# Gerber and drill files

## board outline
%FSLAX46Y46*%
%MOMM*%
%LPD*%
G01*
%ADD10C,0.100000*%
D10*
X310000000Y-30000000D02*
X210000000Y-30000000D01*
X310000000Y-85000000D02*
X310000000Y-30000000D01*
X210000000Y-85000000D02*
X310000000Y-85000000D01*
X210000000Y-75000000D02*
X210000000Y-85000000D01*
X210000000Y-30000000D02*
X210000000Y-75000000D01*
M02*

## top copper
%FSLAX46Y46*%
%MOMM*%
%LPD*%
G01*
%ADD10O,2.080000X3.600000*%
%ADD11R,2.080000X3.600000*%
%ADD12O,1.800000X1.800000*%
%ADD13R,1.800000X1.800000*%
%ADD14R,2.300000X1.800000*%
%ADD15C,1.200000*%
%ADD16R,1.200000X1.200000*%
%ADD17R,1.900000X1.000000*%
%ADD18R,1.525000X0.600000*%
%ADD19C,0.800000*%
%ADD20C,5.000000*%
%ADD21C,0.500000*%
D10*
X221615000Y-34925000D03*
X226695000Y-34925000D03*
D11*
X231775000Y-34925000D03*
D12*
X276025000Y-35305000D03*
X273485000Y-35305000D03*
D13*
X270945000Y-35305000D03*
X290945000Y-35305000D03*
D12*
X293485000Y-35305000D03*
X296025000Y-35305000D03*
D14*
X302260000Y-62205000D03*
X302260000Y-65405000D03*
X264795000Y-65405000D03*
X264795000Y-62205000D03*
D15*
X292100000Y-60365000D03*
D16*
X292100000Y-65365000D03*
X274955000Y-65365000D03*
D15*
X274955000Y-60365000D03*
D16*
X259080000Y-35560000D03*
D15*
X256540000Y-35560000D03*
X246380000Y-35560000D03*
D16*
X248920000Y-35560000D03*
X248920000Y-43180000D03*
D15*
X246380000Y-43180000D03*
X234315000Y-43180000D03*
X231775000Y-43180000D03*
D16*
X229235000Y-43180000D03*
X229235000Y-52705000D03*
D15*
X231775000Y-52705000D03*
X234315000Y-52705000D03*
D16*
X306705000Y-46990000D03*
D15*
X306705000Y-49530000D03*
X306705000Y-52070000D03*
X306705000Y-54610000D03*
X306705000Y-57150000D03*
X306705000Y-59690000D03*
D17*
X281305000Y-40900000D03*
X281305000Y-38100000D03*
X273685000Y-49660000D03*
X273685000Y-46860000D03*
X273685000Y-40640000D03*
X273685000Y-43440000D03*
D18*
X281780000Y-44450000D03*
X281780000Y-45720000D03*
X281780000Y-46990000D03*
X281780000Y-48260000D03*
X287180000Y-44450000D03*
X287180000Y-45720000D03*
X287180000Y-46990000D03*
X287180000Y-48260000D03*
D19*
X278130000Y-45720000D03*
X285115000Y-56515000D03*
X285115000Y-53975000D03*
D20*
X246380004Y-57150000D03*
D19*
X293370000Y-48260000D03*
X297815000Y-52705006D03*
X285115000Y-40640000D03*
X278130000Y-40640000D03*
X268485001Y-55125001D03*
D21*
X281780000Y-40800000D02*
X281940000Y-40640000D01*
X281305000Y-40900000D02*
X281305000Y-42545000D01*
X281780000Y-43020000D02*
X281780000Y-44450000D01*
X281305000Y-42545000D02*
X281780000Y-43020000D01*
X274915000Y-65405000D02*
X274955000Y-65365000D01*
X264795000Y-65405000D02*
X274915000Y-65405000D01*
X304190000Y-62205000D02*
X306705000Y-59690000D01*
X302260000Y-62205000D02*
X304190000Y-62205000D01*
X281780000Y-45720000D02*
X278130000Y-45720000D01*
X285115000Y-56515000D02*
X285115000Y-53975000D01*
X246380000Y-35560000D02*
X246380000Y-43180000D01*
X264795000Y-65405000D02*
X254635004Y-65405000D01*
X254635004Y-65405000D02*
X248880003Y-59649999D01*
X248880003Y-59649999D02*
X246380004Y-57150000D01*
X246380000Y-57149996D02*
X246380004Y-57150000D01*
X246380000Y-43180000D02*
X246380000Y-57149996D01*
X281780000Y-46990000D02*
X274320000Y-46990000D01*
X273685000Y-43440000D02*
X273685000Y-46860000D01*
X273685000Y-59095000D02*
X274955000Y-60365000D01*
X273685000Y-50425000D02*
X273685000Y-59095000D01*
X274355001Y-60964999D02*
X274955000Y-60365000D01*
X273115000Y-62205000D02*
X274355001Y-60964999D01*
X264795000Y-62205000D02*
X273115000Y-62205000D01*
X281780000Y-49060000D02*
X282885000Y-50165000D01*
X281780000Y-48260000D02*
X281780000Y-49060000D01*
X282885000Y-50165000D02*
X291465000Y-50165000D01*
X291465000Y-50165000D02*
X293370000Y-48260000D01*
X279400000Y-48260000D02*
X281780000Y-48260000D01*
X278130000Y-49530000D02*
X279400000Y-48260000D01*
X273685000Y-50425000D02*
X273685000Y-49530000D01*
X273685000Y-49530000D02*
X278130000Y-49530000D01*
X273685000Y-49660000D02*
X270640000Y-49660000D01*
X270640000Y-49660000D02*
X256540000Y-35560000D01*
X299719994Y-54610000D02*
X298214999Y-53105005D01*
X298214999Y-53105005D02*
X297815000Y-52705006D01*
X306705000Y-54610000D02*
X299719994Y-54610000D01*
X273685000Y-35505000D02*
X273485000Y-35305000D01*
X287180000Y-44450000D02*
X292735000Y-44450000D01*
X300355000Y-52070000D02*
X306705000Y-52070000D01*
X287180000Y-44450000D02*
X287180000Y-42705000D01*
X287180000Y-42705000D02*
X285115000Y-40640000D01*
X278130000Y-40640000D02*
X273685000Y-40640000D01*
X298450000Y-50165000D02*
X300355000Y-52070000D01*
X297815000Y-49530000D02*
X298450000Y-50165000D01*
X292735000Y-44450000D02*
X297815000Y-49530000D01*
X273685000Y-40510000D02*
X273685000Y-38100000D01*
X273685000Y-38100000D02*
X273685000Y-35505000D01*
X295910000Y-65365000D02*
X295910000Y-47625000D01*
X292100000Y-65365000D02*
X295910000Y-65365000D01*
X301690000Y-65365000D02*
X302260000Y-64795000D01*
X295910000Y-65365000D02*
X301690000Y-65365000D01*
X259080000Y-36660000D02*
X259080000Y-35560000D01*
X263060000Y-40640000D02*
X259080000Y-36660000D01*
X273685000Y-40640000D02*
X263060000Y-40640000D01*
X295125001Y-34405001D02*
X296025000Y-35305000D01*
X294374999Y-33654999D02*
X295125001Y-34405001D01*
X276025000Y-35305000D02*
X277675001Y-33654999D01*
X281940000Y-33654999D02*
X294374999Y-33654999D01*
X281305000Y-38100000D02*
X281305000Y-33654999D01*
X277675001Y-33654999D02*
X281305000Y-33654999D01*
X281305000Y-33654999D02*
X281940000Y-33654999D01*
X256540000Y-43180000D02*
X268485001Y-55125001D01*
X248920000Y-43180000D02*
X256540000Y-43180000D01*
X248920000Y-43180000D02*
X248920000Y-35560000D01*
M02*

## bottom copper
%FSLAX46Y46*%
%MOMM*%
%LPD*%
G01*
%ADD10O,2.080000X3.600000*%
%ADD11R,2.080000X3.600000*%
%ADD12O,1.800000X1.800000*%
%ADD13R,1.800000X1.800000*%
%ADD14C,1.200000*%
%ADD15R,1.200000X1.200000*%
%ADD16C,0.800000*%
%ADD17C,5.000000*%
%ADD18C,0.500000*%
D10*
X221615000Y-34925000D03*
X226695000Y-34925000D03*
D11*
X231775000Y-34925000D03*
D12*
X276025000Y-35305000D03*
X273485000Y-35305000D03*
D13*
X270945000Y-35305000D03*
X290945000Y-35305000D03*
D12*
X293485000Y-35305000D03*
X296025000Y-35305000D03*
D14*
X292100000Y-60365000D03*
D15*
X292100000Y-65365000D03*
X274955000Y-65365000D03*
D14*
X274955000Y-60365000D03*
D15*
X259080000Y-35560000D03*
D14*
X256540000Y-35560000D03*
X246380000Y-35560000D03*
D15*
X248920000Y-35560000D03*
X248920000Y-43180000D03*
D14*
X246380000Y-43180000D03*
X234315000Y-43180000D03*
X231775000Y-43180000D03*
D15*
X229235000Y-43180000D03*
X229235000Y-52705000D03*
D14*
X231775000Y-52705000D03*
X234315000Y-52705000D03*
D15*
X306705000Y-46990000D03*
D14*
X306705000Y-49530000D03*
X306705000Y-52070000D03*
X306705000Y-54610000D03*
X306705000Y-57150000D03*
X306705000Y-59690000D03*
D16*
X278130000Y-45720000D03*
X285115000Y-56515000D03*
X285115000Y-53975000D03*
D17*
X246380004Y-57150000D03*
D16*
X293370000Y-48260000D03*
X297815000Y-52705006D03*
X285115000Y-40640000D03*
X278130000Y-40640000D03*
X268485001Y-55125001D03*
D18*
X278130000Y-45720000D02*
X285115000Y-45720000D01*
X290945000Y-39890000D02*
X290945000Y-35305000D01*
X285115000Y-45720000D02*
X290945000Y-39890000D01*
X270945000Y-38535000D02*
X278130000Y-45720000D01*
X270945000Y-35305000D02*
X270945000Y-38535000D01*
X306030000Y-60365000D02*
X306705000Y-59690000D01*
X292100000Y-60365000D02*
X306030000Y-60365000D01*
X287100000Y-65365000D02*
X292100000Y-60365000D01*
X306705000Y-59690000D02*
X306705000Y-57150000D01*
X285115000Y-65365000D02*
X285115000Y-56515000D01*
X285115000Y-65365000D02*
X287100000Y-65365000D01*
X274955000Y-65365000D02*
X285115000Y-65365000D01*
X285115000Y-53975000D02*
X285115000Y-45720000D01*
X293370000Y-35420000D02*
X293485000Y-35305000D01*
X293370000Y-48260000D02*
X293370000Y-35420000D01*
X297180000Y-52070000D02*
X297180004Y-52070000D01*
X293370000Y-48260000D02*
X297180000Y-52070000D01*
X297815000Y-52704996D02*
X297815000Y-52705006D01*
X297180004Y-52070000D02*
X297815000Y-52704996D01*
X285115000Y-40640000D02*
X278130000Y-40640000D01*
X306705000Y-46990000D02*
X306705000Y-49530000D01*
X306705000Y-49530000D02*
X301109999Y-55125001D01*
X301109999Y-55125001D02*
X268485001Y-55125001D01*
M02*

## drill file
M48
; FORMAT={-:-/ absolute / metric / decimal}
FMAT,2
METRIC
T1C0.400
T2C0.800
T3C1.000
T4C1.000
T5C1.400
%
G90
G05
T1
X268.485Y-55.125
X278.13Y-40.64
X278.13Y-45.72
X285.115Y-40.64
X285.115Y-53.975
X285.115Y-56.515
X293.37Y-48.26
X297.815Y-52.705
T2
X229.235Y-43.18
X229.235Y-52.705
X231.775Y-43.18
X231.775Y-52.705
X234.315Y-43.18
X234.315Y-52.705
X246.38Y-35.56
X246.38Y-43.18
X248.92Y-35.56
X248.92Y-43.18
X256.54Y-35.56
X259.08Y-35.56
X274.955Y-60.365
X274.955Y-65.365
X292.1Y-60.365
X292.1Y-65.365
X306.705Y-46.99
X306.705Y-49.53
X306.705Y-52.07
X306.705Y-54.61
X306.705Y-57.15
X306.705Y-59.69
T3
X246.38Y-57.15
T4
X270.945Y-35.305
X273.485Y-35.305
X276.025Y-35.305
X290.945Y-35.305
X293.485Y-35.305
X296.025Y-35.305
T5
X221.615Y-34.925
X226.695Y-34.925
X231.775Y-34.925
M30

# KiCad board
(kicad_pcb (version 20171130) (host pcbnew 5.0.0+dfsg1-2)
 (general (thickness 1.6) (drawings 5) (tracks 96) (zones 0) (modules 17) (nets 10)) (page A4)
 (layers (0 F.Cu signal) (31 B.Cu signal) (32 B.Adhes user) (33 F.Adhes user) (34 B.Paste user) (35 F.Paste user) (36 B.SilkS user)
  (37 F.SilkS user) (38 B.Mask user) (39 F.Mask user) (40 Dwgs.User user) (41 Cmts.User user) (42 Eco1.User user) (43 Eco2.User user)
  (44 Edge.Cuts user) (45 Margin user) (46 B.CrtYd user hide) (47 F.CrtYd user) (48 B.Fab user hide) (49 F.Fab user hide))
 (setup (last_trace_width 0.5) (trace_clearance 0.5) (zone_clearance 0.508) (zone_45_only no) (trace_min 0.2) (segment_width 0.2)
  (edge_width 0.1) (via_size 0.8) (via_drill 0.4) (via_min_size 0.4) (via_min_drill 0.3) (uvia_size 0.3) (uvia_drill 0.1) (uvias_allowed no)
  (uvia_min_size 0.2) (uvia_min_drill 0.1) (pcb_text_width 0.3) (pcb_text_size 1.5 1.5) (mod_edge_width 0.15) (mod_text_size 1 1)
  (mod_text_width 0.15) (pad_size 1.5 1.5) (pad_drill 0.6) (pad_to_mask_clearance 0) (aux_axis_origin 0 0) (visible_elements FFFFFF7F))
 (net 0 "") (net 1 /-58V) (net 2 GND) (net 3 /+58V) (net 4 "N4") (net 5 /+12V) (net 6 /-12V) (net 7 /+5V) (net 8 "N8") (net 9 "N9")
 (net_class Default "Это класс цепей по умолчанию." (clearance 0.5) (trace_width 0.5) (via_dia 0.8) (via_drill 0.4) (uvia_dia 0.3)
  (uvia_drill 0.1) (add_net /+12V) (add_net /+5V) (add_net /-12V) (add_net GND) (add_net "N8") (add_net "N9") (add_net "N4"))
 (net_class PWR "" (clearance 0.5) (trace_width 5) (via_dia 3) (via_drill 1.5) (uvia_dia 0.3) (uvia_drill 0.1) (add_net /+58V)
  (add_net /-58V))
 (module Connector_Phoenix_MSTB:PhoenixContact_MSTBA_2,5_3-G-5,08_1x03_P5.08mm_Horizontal (layer F.Cu) (at 231.775 34.925 180)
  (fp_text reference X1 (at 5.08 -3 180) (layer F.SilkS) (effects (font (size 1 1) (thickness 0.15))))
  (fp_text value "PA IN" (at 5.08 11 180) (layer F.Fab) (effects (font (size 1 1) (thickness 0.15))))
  (pad 3 thru_hole oval (at 10.16 0 180) (size 2.08 3.6) (drill 1.4) (layers *.Cu *.Mask) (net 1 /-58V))
  (pad 2 thru_hole oval (at 5.08 0 180) (size 2.08 3.6) (drill 1.4) (layers *.Cu *.Mask) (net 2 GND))
  (pad 1 thru_hole rect (at 0 0 180) (size 2.08 3.6) (drill 1.4) (layers *.Cu *.Mask) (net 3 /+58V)))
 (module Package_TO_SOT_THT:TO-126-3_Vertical (layer F.Cu) (at 270.945 35.305)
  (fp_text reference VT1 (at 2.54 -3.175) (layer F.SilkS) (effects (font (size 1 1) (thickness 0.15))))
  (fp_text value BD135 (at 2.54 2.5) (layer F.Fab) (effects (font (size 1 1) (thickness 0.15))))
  (pad 3 thru_hole oval (at 5.08 0) (size 1.8 1.8) (drill 1) (layers *.Cu *.Mask) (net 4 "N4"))
  (pad 2 thru_hole oval (at 2.54 0) (size 1.8 1.8) (drill 1) (layers *.Cu *.Mask) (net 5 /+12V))
  (pad 1 thru_hole rect (at 0 0) (size 1.8 1.8) (drill 1) (layers *.Cu *.Mask) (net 2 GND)))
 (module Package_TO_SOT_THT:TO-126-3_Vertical (layer F.Cu) (at 290.945 35.305)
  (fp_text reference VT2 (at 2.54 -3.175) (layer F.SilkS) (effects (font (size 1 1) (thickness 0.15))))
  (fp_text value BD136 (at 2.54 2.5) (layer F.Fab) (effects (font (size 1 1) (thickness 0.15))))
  (pad 1 thru_hole rect (at 0 0) (size 1.8 1.8) (drill 1) (layers *.Cu *.Mask) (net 2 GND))
  (pad 2 thru_hole oval (at 2.54 0) (size 1.8 1.8) (drill 1) (layers *.Cu *.Mask) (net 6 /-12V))
  (pad 3 thru_hole oval (at 5.08 0) (size 1.8 1.8) (drill 1) (layers *.Cu *.Mask) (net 4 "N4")))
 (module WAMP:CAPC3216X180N (layer F.Cu) (at 302.26 63.805 180)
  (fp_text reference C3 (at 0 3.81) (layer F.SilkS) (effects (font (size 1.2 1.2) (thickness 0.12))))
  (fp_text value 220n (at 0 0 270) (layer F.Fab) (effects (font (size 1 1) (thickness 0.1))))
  (pad 2 smd rect (at 0 1.6 180) (size 2.3 1.8) (layers F.Cu F.Paste F.Mask) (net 2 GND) (solder_mask_margin 0.2))
  (pad 1 smd rect (at 0 -1.6 180) (size 2.3 1.8) (layers F.Cu F.Paste F.Mask) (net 5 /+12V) (solder_mask_margin 0.2)))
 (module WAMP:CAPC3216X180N (layer F.Cu) (at 264.795 63.805 180)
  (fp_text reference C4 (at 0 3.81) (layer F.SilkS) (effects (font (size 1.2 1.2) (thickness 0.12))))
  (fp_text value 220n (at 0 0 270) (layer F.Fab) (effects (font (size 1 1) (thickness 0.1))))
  (pad 1 smd rect (at 0 -1.6 180) (size 2.3 1.8) (layers F.Cu F.Paste F.Mask) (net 2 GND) (solder_mask_margin 0.2))
  (pad 2 smd rect (at 0 1.6 180) (size 2.3 1.8) (layers F.Cu F.Paste F.Mask) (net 6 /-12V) (solder_mask_margin 0.2)))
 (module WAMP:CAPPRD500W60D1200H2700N (layer F.Cu) (at 292.1 62.865 180)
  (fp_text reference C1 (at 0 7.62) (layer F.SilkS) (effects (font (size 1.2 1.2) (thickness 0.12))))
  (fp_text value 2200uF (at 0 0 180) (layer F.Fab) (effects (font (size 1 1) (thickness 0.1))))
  (pad 2 thru_hole circle (at 0 2.5 180) (size 1.2 1.2) (drill 0.8) (layers F&B.Cu *.Paste *.Mask) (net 2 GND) (solder_mask_margin 0.2))
  (pad 1 thru_hole rect (at 0 -2.5 180) (size 1.2 1.2) (drill 0.8) (layers F&B.Cu *.Paste *.Mask) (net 5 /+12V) (solder_mask_margin 0.2)))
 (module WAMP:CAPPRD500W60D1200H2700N (layer F.Cu) (at 274.955 62.865 180)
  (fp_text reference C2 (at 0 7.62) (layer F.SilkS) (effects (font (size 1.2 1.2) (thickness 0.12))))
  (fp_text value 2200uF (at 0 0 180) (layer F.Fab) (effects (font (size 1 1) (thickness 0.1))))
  (pad 1 thru_hole rect (at 0 -2.5 180) (size 1.2 1.2) (drill 0.8) (layers F&B.Cu *.Paste *.Mask) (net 2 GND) (solder_mask_margin 0.2))
  (pad 2 thru_hole circle (at 0 2.5 180) (size 1.2 1.2) (drill 0.8) (layers F&B.Cu *.Paste *.Mask) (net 6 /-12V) (solder_mask_margin 0.2)))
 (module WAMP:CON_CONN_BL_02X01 (layer F.Cu) (at 257.81 35.56 270)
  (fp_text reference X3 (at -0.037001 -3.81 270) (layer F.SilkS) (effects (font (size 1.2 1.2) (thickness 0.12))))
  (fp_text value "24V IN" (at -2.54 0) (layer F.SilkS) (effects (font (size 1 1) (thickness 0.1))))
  (pad 1 thru_hole rect (at 0 -1.27 270) (size 1.2 1.2) (drill 0.8) (layers F&B.Cu *.Paste *.Mask) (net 5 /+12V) (solder_mask_margin 0.2))
  (pad 2 thru_hole circle (at 0 1.27 270) (size 1.2 1.2) (drill 0.8) (layers F&B.Cu *.Paste *.Mask) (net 6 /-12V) (solder_mask_margin 0.2)))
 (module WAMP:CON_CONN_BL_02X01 (layer F.Cu) (at 247.65 35.56 270)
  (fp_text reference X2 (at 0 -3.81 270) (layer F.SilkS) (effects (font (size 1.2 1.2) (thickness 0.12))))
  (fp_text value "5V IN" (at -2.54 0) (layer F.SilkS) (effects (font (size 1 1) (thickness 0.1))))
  (pad 2 thru_hole circle (at 0 1.27 270) (size 1.2 1.2) (drill 0.8) (layers F&B.Cu *.Paste *.Mask) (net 2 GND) (solder_mask_margin 0.2))
  (pad 1 thru_hole rect (at 0 -1.27 270) (size 1.2 1.2) (drill 0.8) (layers F&B.Cu *.Paste *.Mask) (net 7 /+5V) (solder_mask_margin 0.2)))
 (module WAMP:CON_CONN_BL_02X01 (layer F.Cu) (at 247.65 43.18 270)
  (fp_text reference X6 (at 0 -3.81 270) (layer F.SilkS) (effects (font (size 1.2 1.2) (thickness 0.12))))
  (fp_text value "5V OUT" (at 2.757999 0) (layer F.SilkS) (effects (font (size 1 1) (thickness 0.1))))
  (pad 1 thru_hole rect (at 0 -1.27 270) (size 1.2 1.2) (drill 0.8) (layers F&B.Cu *.Paste *.Mask) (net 7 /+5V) (solder_mask_margin 0.2))
  (pad 2 thru_hole circle (at 0 1.27 270) (size 1.2 1.2) (drill 0.8) (layers F&B.Cu *.Paste *.Mask) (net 2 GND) (solder_mask_margin 0.2)))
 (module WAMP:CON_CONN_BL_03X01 (layer F.Cu) (at 231.775 43.18 90)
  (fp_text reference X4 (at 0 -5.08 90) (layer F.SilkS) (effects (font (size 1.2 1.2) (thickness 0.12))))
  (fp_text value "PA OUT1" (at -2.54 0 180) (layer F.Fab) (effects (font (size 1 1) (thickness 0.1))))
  (pad 3 thru_hole circle (at 0 2.54 90) (size 1.2 1.2) (drill 0.8) (layers F&B.Cu *.Paste *.Mask) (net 1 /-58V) (solder_mask_margin 0.2))
  (pad 2 thru_hole circle (at 0 0 90) (size 1.2 1.2) (drill 0.8) (layers F&B.Cu *.Paste *.Mask) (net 2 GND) (solder_mask_margin 0.2))
  (pad 1 thru_hole rect (at 0 -2.54 90) (size 1.2 1.2) (drill 0.8) (layers F&B.Cu *.Paste *.Mask) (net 3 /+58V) (solder_mask_margin 0.2)))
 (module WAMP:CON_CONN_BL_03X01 (layer F.Cu) (at 231.775 52.705 90)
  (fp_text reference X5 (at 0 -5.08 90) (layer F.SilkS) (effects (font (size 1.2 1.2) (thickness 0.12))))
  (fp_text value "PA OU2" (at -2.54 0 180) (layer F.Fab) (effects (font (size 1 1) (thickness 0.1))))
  (pad 1 thru_hole rect (at 0 -2.54 90) (size 1.2 1.2) (drill 0.8) (layers F&B.Cu *.Paste *.Mask) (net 3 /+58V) (solder_mask_margin 0.2))
  (pad 2 thru_hole circle (at 0 0 90) (size 1.2 1.2) (drill 0.8) (layers F&B.Cu *.Paste *.Mask) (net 2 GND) (solder_mask_margin 0.2))
  (pad 3 thru_hole circle (at 0 2.54 90) (size 1.2 1.2) (drill 0.8) (layers F&B.Cu *.Paste *.Mask) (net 1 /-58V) (solder_mask_margin 0.2)))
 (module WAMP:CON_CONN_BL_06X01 (layer F.Cu) (at 306.705 53.34)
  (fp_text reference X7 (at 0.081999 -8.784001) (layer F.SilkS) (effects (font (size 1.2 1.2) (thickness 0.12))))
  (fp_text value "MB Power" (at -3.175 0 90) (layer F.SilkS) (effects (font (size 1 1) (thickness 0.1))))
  (pad 1 thru_hole rect (at 0 -6.35) (size 1.2 1.2) (drill 0.8) (layers F&B.Cu *.Paste *.Mask) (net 7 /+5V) (solder_mask_margin 0.2))
  (pad 2 thru_hole circle (at 0 -3.81) (size 1.2 1.2) (drill 0.8) (layers F&B.Cu *.Paste *.Mask) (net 7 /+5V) (solder_mask_margin 0.2))
  (pad 3 thru_hole circle (at 0 -1.27) (size 1.2 1.2) (drill 0.8) (layers F&B.Cu *.Paste *.Mask) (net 5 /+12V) (solder_mask_margin 0.2))
  (pad 4 thru_hole circle (at 0 1.27) (size 1.2 1.2) (drill 0.8) (layers F&B.Cu *.Paste *.Mask) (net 6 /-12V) (solder_mask_margin 0.2))
  (pad 5 thru_hole circle (at 0 3.81) (size 1.2 1.2) (drill 0.8) (layers F&B.Cu *.Paste *.Mask) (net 2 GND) (solder_mask_margin 0.2))
  (pad 6 thru_hole circle (at 0 6.35) (size 1.2 1.2) (drill 0.8) (layers F&B.Cu *.Paste *.Mask) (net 2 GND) (solder_mask_margin 0.2)))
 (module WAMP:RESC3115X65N (layer F.Cu) (at 281.305 39.5 180)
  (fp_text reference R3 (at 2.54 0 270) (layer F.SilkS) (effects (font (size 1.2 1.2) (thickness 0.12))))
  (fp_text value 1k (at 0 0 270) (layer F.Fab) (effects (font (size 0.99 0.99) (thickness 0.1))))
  (pad 1 smd rect (at 0 -1.4 180) (size 1.9 1) (layers F.Cu F.Paste F.Mask) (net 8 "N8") (solder_mask_margin 0.2))
  (pad 2 smd rect (at 0 1.4 180) (size 1.9 1) (layers F.Cu F.Paste F.Mask) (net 4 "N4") (solder_mask_margin 0.2)))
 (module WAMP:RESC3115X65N (layer F.Cu) (at 273.685 48.26)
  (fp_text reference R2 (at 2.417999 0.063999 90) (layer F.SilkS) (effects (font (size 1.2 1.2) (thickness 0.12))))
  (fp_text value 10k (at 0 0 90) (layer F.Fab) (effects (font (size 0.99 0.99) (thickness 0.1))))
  (pad 2 smd rect (at 0 1.4) (size 1.9 1) (layers F.Cu F.Paste F.Mask) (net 6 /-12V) (solder_mask_margin 0.2))
  (pad 1 smd rect (at 0 -1.4) (size 1.9 1) (layers F.Cu F.Paste F.Mask) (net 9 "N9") (solder_mask_margin 0.2)))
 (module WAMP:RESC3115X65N (layer F.Cu) (at 273.685 42.04)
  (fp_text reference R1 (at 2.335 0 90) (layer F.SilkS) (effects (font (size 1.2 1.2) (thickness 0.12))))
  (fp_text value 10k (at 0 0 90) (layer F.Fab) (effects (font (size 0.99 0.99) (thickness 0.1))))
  (pad 1 smd rect (at 0 -1.4) (size 1.9 1) (layers F.Cu F.Paste F.Mask) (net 5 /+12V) (solder_mask_margin 0.2))
  (pad 2 smd rect (at 0 1.4) (size 1.9 1) (layers F.Cu F.Paste F.Mask) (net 9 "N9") (solder_mask_margin 0.2)))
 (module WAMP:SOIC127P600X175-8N (layer F.Cu) (at 284.48 46.355)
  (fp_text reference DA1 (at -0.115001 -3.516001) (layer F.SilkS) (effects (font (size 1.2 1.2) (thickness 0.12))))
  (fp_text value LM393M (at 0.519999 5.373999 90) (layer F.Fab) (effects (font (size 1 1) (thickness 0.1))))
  (pad 1 smd rect (at -2.7 -1.905) (size 1.525 0.6) (layers F.Cu F.Paste F.Mask) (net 8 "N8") (solder_mask_margin 0.2))
  (pad 2 smd rect (at -2.7 -0.635) (size 1.525 0.6) (layers F.Cu F.Paste F.Mask) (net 2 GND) (solder_mask_margin 0.2))
  (pad 3 smd rect (at -2.7 0.635) (size 1.525 0.6) (layers F.Cu F.Paste F.Mask) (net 9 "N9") (solder_mask_margin 0.2))
  (pad 4 smd rect (at -2.7 1.905) (size 1.525 0.6) (layers F.Cu F.Paste F.Mask) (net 6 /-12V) (solder_mask_margin 0.2))
  (pad 8 smd rect (at 2.7 -1.905) (size 1.525 0.6) (layers F.Cu F.Paste F.Mask) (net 5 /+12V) (solder_mask_margin 0.2))
  (pad 7 smd rect (at 2.7 -0.635) (size 1.525 0.6) (layers F.Cu F.Paste F.Mask) (solder_mask_margin 0.2))
  (pad 6 smd rect (at 2.7 0.635) (size 1.525 0.6) (layers F.Cu F.Paste F.Mask) (solder_mask_margin 0.2))
  (pad 5 smd rect (at 2.7 1.905) (size 1.525 0.6) (layers F.Cu F.Paste F.Mask) (solder_mask_margin 0.2)))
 (gr_line (start 310 30) (end 210 30) (layer Edge.Cuts) (width 0.1))
 (gr_line (start 310 85) (end 310 30) (layer Edge.Cuts) (width 0.1))
 (gr_line (start 210 85) (end 310 85) (layer Edge.Cuts) (width 0.1))
 (gr_line (start 210 75) (end 210 85) (layer Edge.Cuts) (width 0.1))
 (gr_line (start 210 30) (end 210 75) (layer Edge.Cuts) (width 0.1))
 (segment (start 281.78 40.8) (end 281.94 40.64) (width 0.5) (layer F.Cu) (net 8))
 (segment (start 281.305 40.9) (end 281.305 42.545) (width 0.5) (layer F.Cu) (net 8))
 (segment (start 281.78 43.02) (end 281.78 44.45) (width 0.5) (layer F.Cu) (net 8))
 (segment (start 281.305 42.545) (end 281.78 43.02) (width 0.5) (layer F.Cu) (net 8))
 (segment (start 274.915 65.405) (end 274.955 65.365) (width 0.5) (layer F.Cu) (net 2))
 (segment (start 264.795 65.405) (end 274.915 65.405) (width 0.5) (layer F.Cu) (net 2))
 (segment (start 304.19 62.205) (end 306.705 59.69) (width 0.5) (layer F.Cu) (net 2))
 (segment (start 302.26 62.205) (end 304.19 62.205) (width 0.5) (layer F.Cu) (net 2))
 (via (at 278.13 45.72) (size 0.8) (drill 0.4) (layers F.Cu B.Cu) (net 2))
 (segment (start 281.78 45.72) (end 278.13 45.72) (width 0.5) (layer F.Cu) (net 2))
 (segment (start 278.13 45.72) (end 285.115 45.72) (width 0.5) (layer B.Cu) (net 2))
 (segment (start 290.945 39.89) (end 290.945 35.305) (width 0.5) (layer B.Cu) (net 2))
 (segment (start 285.115 45.72) (end 290.945 39.89) (width 0.5) (layer B.Cu) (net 2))
 (segment (start 270.945 38.535) (end 278.13 45.72) (width 0.5) (layer B.Cu) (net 2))
 (segment (start 270.945 35.305) (end 270.945 38.535) (width 0.5) (layer B.Cu) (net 2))
 (segment (start 306.03 60.365) (end 306.705 59.69) (width 0.5) (layer B.Cu) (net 2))
 (segment (start 292.1 60.365) (end 306.03 60.365) (width 0.5) (layer B.Cu) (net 2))
 (segment (start 287.1 65.365) (end 292.1 60.365) (width 0.5) (layer B.Cu) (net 2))
 (segment (start 306.705 59.69) (end 306.705 57.15) (width 0.5) (layer B.Cu) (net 2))
 (segment (start 285.115 65.365) (end 285.115 56.515) (width 0.5) (layer B.Cu) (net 2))
 (segment (start 285.115 65.365) (end 287.1 65.365) (width 0.5) (layer B.Cu) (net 2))
 (via (at 285.115 56.515) (size 0.8) (drill 0.4) (layers F.Cu B.Cu) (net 2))
 (segment (start 274.955 65.365) (end 285.115 65.365) (width 0.5) (layer B.Cu) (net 2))
 (via (at 285.115 53.975) (size 0.8) (drill 0.4) (layers F.Cu B.Cu) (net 2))
 (segment (start 285.115 56.515) (end 285.115 53.975) (width 0.5) (layer F.Cu) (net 2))
 (segment (start 285.115 53.975) (end 285.115 45.72) (width 0.5) (layer B.Cu) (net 2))
 (segment (start 246.38 35.56) (end 246.38 43.18) (width 0.5) (layer F.Cu) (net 2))
 (via (at 246.380004 57.15) (size 5) (drill 1) (layers F.Cu B.Cu) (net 2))
 (segment (start 264.795 65.405) (end 254.635004 65.405) (width 0.5) (layer F.Cu) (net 2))
 (segment (start 254.635004 65.405) (end 248.880003 59.649999) (width 0.5) (layer F.Cu) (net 2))
 (segment (start 248.880003 59.649999) (end 246.380004 57.15) (width 0.5) (layer F.Cu) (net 2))
 (segment (start 246.38 57.149996) (end 246.380004 57.15) (width 0.5) (layer F.Cu) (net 2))
 (segment (start 246.38 43.18) (end 246.38 57.149996) (width 0.5) (layer F.Cu) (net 2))
 (segment (start 281.78 46.99) (end 274.32 46.99) (width 0.5) (layer F.Cu) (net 9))
 (segment (start 273.685 43.44) (end 273.685 46.86) (width 0.5) (layer F.Cu) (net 9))
 (segment (start 273.685 59.095) (end 274.955 60.365) (width 0.5) (layer F.Cu) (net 6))
 (segment (start 273.685 50.425) (end 273.685 59.095) (width 0.5) (layer F.Cu) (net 6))
 (segment (start 274.355001 60.964999) (end 274.955 60.365) (width 0.5) (layer F.Cu) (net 6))
 (segment (start 273.115 62.205) (end 274.355001 60.964999) (width 0.5) (layer F.Cu) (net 6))
 (segment (start 264.795 62.205) (end 273.115 62.205) (width 0.5) (layer F.Cu) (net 6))
 (segment (start 281.78 49.06) (end 282.885 50.165) (width 0.5) (layer F.Cu) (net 6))
 (segment (start 281.78 48.26) (end 281.78 49.06) (width 0.5) (layer F.Cu) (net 6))
 (segment (start 282.885 50.165) (end 291.465 50.165) (width 0.5) (layer F.Cu) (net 6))
 (via (at 293.37 48.26) (size 0.8) (drill 0.4) (layers F.Cu B.Cu) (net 6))
 (segment (start 291.465 50.165) (end 293.37 48.26) (width 0.5) (layer F.Cu) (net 6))
 (segment (start 293.37 35.42) (end 293.485 35.305) (width 0.5) (layer B.Cu) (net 6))
 (segment (start 293.37 48.26) (end 293.37 35.42) (width 0.5) (layer B.Cu) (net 6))
 (segment (start 279.4 48.26) (end 281.78 48.26) (width 0.5) (layer F.Cu) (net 6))
 (segment (start 278.13 49.53) (end 279.4 48.26) (width 0.5) (layer F.Cu) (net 6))
 (segment (start 273.685 50.425) (end 273.685 49.53) (width 0.5) (layer F.Cu) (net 6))
 (segment (start 273.685 49.53) (end 278.13 49.53) (width 0.5) (layer F.Cu) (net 6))
 (segment (start 273.685 49.66) (end 270.64 49.66) (width 0.5) (layer F.Cu) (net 6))
 (segment (start 270.64 49.66) (end 256.54 35.56) (width 0.5) (layer F.Cu) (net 6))
 (segment (start 297.18 52.07) (end 297.180004 52.07) (width 0.5) (layer B.Cu) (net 6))
 (segment (start 293.37 48.26) (end 297.18 52.07) (width 0.5) (layer B.Cu) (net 6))
 (segment (start 299.719994 54.61) (end 298.214999 53.105005) (width 0.5) (layer F.Cu) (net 6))
 (segment (start 298.214999 53.105005) (end 297.815 52.705006) (width 0.5) (layer F.Cu) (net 6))
 (via (at 297.815 52.705006) (size 0.8) (drill 0.4) (layers F.Cu B.Cu) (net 6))
 (segment (start 306.705 54.61) (end 299.719994 54.61) (width 0.5) (layer F.Cu) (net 6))
 (segment (start 297.815 52.704996) (end 297.815 52.705006) (width 0.5) (layer B.Cu) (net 6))
 (segment (start 297.180004 52.07) (end 297.815 52.704996) (width 0.5) (layer B.Cu) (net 6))
 (segment (start 273.685 35.505) (end 273.485 35.305) (width 0.5) (layer F.Cu) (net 5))
 (segment (start 287.18 44.45) (end 292.735 44.45) (width 0.5) (layer F.Cu) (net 5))
 (segment (start 300.355 52.07) (end 306.705 52.07) (width 0.5) (layer F.Cu) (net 5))
 (via (at 285.115 40.64) (size 0.8) (drill 0.4) (layers F.Cu B.Cu) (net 5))
 (segment (start 287.18 44.45) (end 287.18 42.705) (width 0.5) (layer F.Cu) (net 5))
 (segment (start 287.18 42.705) (end 285.115 40.64) (width 0.5) (layer F.Cu) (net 5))
 (via (at 278.13 40.64) (size 0.8) (drill 0.4) (layers F.Cu B.Cu) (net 5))
 (segment (start 285.115 40.64) (end 278.13 40.64) (width 0.5) (layer B.Cu) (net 5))
 (segment (start 278.13 40.64) (end 273.685 40.64) (width 0.5) (layer F.Cu) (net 5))
 (segment (start 298.45 50.165) (end 300.355 52.07) (width 0.5) (layer F.Cu) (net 5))
 (segment (start 297.815 49.53) (end 298.45 50.165) (width 0.5) (layer F.Cu) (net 5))
 (segment (start 292.735 44.45) (end 297.815 49.53) (width 0.5) (layer F.Cu) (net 5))
 (segment (start 273.685 40.51) (end 273.685 38.1) (width 0.5) (layer F.Cu) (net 5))
 (segment (start 273.685 38.1) (end 273.685 35.505) (width 0.5) (layer F.Cu) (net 5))
 (segment (start 295.91 65.365) (end 295.91 47.625) (width 0.5) (layer F.Cu) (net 5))
 (segment (start 292.1 65.365) (end 295.91 65.365) (width 0.5) (layer F.Cu) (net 5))
 (segment (start 301.69 65.365) (end 302.26 64.795) (width 0.5) (layer F.Cu) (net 5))
 (segment (start 295.91 65.365) (end 301.69 65.365) (width 0.5) (layer F.Cu) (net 5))
 (segment (start 259.08 36.66) (end 259.08 35.56) (width 0.5) (layer F.Cu) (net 5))
 (segment (start 263.06 40.64) (end 259.08 36.66) (width 0.5) (layer F.Cu) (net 5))
 (segment (start 273.685 40.64) (end 263.06 40.64) (width 0.5) (layer F.Cu) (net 5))
 (segment (start 295.125001 34.405001) (end 296.025 35.305) (width 0.5) (layer F.Cu) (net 4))
 (segment (start 294.374999 33.654999) (end 295.125001 34.405001) (width 0.5) (layer F.Cu) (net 4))
 (segment (start 276.025 35.305) (end 277.675001 33.654999) (width 0.5) (layer F.Cu) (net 4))
 (segment (start 281.94 33.654999) (end 294.374999 33.654999) (width 0.5) (layer F.Cu) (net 4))
 (segment (start 281.305 38.1) (end 281.305 33.654999) (width 0.5) (layer F.Cu) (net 4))
 (segment (start 277.675001 33.654999) (end 281.305 33.654999) (width 0.5) (layer F.Cu) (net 4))
 (segment (start 281.305 33.654999) (end 281.94 33.654999) (width 0.5) (layer F.Cu) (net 4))
 (segment (start 306.705 46.99) (end 306.705 49.53) (width 0.5) (layer B.Cu) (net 7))
 (segment (start 306.705 49.53) (end 301.109999 55.125001) (width 0.5) (layer B.Cu) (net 7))
 (segment (start 301.109999 55.125001) (end 268.485001 55.125001) (width 0.5) (layer B.Cu) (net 7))
 (via (at 268.485001 55.125001) (size 0.8) (drill 0.4) (layers F.Cu B.Cu) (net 7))
 (segment (start 256.54 43.18) (end 268.485001 55.125001) (width 0.5) (layer F.Cu) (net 7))
 (segment (start 248.92 43.18) (end 256.54 43.18) (width 0.5) (layer F.Cu) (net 7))
 (segment (start 248.92 43.18) (end 248.92 35.56) (width 0.5) (layer F.Cu) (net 7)))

